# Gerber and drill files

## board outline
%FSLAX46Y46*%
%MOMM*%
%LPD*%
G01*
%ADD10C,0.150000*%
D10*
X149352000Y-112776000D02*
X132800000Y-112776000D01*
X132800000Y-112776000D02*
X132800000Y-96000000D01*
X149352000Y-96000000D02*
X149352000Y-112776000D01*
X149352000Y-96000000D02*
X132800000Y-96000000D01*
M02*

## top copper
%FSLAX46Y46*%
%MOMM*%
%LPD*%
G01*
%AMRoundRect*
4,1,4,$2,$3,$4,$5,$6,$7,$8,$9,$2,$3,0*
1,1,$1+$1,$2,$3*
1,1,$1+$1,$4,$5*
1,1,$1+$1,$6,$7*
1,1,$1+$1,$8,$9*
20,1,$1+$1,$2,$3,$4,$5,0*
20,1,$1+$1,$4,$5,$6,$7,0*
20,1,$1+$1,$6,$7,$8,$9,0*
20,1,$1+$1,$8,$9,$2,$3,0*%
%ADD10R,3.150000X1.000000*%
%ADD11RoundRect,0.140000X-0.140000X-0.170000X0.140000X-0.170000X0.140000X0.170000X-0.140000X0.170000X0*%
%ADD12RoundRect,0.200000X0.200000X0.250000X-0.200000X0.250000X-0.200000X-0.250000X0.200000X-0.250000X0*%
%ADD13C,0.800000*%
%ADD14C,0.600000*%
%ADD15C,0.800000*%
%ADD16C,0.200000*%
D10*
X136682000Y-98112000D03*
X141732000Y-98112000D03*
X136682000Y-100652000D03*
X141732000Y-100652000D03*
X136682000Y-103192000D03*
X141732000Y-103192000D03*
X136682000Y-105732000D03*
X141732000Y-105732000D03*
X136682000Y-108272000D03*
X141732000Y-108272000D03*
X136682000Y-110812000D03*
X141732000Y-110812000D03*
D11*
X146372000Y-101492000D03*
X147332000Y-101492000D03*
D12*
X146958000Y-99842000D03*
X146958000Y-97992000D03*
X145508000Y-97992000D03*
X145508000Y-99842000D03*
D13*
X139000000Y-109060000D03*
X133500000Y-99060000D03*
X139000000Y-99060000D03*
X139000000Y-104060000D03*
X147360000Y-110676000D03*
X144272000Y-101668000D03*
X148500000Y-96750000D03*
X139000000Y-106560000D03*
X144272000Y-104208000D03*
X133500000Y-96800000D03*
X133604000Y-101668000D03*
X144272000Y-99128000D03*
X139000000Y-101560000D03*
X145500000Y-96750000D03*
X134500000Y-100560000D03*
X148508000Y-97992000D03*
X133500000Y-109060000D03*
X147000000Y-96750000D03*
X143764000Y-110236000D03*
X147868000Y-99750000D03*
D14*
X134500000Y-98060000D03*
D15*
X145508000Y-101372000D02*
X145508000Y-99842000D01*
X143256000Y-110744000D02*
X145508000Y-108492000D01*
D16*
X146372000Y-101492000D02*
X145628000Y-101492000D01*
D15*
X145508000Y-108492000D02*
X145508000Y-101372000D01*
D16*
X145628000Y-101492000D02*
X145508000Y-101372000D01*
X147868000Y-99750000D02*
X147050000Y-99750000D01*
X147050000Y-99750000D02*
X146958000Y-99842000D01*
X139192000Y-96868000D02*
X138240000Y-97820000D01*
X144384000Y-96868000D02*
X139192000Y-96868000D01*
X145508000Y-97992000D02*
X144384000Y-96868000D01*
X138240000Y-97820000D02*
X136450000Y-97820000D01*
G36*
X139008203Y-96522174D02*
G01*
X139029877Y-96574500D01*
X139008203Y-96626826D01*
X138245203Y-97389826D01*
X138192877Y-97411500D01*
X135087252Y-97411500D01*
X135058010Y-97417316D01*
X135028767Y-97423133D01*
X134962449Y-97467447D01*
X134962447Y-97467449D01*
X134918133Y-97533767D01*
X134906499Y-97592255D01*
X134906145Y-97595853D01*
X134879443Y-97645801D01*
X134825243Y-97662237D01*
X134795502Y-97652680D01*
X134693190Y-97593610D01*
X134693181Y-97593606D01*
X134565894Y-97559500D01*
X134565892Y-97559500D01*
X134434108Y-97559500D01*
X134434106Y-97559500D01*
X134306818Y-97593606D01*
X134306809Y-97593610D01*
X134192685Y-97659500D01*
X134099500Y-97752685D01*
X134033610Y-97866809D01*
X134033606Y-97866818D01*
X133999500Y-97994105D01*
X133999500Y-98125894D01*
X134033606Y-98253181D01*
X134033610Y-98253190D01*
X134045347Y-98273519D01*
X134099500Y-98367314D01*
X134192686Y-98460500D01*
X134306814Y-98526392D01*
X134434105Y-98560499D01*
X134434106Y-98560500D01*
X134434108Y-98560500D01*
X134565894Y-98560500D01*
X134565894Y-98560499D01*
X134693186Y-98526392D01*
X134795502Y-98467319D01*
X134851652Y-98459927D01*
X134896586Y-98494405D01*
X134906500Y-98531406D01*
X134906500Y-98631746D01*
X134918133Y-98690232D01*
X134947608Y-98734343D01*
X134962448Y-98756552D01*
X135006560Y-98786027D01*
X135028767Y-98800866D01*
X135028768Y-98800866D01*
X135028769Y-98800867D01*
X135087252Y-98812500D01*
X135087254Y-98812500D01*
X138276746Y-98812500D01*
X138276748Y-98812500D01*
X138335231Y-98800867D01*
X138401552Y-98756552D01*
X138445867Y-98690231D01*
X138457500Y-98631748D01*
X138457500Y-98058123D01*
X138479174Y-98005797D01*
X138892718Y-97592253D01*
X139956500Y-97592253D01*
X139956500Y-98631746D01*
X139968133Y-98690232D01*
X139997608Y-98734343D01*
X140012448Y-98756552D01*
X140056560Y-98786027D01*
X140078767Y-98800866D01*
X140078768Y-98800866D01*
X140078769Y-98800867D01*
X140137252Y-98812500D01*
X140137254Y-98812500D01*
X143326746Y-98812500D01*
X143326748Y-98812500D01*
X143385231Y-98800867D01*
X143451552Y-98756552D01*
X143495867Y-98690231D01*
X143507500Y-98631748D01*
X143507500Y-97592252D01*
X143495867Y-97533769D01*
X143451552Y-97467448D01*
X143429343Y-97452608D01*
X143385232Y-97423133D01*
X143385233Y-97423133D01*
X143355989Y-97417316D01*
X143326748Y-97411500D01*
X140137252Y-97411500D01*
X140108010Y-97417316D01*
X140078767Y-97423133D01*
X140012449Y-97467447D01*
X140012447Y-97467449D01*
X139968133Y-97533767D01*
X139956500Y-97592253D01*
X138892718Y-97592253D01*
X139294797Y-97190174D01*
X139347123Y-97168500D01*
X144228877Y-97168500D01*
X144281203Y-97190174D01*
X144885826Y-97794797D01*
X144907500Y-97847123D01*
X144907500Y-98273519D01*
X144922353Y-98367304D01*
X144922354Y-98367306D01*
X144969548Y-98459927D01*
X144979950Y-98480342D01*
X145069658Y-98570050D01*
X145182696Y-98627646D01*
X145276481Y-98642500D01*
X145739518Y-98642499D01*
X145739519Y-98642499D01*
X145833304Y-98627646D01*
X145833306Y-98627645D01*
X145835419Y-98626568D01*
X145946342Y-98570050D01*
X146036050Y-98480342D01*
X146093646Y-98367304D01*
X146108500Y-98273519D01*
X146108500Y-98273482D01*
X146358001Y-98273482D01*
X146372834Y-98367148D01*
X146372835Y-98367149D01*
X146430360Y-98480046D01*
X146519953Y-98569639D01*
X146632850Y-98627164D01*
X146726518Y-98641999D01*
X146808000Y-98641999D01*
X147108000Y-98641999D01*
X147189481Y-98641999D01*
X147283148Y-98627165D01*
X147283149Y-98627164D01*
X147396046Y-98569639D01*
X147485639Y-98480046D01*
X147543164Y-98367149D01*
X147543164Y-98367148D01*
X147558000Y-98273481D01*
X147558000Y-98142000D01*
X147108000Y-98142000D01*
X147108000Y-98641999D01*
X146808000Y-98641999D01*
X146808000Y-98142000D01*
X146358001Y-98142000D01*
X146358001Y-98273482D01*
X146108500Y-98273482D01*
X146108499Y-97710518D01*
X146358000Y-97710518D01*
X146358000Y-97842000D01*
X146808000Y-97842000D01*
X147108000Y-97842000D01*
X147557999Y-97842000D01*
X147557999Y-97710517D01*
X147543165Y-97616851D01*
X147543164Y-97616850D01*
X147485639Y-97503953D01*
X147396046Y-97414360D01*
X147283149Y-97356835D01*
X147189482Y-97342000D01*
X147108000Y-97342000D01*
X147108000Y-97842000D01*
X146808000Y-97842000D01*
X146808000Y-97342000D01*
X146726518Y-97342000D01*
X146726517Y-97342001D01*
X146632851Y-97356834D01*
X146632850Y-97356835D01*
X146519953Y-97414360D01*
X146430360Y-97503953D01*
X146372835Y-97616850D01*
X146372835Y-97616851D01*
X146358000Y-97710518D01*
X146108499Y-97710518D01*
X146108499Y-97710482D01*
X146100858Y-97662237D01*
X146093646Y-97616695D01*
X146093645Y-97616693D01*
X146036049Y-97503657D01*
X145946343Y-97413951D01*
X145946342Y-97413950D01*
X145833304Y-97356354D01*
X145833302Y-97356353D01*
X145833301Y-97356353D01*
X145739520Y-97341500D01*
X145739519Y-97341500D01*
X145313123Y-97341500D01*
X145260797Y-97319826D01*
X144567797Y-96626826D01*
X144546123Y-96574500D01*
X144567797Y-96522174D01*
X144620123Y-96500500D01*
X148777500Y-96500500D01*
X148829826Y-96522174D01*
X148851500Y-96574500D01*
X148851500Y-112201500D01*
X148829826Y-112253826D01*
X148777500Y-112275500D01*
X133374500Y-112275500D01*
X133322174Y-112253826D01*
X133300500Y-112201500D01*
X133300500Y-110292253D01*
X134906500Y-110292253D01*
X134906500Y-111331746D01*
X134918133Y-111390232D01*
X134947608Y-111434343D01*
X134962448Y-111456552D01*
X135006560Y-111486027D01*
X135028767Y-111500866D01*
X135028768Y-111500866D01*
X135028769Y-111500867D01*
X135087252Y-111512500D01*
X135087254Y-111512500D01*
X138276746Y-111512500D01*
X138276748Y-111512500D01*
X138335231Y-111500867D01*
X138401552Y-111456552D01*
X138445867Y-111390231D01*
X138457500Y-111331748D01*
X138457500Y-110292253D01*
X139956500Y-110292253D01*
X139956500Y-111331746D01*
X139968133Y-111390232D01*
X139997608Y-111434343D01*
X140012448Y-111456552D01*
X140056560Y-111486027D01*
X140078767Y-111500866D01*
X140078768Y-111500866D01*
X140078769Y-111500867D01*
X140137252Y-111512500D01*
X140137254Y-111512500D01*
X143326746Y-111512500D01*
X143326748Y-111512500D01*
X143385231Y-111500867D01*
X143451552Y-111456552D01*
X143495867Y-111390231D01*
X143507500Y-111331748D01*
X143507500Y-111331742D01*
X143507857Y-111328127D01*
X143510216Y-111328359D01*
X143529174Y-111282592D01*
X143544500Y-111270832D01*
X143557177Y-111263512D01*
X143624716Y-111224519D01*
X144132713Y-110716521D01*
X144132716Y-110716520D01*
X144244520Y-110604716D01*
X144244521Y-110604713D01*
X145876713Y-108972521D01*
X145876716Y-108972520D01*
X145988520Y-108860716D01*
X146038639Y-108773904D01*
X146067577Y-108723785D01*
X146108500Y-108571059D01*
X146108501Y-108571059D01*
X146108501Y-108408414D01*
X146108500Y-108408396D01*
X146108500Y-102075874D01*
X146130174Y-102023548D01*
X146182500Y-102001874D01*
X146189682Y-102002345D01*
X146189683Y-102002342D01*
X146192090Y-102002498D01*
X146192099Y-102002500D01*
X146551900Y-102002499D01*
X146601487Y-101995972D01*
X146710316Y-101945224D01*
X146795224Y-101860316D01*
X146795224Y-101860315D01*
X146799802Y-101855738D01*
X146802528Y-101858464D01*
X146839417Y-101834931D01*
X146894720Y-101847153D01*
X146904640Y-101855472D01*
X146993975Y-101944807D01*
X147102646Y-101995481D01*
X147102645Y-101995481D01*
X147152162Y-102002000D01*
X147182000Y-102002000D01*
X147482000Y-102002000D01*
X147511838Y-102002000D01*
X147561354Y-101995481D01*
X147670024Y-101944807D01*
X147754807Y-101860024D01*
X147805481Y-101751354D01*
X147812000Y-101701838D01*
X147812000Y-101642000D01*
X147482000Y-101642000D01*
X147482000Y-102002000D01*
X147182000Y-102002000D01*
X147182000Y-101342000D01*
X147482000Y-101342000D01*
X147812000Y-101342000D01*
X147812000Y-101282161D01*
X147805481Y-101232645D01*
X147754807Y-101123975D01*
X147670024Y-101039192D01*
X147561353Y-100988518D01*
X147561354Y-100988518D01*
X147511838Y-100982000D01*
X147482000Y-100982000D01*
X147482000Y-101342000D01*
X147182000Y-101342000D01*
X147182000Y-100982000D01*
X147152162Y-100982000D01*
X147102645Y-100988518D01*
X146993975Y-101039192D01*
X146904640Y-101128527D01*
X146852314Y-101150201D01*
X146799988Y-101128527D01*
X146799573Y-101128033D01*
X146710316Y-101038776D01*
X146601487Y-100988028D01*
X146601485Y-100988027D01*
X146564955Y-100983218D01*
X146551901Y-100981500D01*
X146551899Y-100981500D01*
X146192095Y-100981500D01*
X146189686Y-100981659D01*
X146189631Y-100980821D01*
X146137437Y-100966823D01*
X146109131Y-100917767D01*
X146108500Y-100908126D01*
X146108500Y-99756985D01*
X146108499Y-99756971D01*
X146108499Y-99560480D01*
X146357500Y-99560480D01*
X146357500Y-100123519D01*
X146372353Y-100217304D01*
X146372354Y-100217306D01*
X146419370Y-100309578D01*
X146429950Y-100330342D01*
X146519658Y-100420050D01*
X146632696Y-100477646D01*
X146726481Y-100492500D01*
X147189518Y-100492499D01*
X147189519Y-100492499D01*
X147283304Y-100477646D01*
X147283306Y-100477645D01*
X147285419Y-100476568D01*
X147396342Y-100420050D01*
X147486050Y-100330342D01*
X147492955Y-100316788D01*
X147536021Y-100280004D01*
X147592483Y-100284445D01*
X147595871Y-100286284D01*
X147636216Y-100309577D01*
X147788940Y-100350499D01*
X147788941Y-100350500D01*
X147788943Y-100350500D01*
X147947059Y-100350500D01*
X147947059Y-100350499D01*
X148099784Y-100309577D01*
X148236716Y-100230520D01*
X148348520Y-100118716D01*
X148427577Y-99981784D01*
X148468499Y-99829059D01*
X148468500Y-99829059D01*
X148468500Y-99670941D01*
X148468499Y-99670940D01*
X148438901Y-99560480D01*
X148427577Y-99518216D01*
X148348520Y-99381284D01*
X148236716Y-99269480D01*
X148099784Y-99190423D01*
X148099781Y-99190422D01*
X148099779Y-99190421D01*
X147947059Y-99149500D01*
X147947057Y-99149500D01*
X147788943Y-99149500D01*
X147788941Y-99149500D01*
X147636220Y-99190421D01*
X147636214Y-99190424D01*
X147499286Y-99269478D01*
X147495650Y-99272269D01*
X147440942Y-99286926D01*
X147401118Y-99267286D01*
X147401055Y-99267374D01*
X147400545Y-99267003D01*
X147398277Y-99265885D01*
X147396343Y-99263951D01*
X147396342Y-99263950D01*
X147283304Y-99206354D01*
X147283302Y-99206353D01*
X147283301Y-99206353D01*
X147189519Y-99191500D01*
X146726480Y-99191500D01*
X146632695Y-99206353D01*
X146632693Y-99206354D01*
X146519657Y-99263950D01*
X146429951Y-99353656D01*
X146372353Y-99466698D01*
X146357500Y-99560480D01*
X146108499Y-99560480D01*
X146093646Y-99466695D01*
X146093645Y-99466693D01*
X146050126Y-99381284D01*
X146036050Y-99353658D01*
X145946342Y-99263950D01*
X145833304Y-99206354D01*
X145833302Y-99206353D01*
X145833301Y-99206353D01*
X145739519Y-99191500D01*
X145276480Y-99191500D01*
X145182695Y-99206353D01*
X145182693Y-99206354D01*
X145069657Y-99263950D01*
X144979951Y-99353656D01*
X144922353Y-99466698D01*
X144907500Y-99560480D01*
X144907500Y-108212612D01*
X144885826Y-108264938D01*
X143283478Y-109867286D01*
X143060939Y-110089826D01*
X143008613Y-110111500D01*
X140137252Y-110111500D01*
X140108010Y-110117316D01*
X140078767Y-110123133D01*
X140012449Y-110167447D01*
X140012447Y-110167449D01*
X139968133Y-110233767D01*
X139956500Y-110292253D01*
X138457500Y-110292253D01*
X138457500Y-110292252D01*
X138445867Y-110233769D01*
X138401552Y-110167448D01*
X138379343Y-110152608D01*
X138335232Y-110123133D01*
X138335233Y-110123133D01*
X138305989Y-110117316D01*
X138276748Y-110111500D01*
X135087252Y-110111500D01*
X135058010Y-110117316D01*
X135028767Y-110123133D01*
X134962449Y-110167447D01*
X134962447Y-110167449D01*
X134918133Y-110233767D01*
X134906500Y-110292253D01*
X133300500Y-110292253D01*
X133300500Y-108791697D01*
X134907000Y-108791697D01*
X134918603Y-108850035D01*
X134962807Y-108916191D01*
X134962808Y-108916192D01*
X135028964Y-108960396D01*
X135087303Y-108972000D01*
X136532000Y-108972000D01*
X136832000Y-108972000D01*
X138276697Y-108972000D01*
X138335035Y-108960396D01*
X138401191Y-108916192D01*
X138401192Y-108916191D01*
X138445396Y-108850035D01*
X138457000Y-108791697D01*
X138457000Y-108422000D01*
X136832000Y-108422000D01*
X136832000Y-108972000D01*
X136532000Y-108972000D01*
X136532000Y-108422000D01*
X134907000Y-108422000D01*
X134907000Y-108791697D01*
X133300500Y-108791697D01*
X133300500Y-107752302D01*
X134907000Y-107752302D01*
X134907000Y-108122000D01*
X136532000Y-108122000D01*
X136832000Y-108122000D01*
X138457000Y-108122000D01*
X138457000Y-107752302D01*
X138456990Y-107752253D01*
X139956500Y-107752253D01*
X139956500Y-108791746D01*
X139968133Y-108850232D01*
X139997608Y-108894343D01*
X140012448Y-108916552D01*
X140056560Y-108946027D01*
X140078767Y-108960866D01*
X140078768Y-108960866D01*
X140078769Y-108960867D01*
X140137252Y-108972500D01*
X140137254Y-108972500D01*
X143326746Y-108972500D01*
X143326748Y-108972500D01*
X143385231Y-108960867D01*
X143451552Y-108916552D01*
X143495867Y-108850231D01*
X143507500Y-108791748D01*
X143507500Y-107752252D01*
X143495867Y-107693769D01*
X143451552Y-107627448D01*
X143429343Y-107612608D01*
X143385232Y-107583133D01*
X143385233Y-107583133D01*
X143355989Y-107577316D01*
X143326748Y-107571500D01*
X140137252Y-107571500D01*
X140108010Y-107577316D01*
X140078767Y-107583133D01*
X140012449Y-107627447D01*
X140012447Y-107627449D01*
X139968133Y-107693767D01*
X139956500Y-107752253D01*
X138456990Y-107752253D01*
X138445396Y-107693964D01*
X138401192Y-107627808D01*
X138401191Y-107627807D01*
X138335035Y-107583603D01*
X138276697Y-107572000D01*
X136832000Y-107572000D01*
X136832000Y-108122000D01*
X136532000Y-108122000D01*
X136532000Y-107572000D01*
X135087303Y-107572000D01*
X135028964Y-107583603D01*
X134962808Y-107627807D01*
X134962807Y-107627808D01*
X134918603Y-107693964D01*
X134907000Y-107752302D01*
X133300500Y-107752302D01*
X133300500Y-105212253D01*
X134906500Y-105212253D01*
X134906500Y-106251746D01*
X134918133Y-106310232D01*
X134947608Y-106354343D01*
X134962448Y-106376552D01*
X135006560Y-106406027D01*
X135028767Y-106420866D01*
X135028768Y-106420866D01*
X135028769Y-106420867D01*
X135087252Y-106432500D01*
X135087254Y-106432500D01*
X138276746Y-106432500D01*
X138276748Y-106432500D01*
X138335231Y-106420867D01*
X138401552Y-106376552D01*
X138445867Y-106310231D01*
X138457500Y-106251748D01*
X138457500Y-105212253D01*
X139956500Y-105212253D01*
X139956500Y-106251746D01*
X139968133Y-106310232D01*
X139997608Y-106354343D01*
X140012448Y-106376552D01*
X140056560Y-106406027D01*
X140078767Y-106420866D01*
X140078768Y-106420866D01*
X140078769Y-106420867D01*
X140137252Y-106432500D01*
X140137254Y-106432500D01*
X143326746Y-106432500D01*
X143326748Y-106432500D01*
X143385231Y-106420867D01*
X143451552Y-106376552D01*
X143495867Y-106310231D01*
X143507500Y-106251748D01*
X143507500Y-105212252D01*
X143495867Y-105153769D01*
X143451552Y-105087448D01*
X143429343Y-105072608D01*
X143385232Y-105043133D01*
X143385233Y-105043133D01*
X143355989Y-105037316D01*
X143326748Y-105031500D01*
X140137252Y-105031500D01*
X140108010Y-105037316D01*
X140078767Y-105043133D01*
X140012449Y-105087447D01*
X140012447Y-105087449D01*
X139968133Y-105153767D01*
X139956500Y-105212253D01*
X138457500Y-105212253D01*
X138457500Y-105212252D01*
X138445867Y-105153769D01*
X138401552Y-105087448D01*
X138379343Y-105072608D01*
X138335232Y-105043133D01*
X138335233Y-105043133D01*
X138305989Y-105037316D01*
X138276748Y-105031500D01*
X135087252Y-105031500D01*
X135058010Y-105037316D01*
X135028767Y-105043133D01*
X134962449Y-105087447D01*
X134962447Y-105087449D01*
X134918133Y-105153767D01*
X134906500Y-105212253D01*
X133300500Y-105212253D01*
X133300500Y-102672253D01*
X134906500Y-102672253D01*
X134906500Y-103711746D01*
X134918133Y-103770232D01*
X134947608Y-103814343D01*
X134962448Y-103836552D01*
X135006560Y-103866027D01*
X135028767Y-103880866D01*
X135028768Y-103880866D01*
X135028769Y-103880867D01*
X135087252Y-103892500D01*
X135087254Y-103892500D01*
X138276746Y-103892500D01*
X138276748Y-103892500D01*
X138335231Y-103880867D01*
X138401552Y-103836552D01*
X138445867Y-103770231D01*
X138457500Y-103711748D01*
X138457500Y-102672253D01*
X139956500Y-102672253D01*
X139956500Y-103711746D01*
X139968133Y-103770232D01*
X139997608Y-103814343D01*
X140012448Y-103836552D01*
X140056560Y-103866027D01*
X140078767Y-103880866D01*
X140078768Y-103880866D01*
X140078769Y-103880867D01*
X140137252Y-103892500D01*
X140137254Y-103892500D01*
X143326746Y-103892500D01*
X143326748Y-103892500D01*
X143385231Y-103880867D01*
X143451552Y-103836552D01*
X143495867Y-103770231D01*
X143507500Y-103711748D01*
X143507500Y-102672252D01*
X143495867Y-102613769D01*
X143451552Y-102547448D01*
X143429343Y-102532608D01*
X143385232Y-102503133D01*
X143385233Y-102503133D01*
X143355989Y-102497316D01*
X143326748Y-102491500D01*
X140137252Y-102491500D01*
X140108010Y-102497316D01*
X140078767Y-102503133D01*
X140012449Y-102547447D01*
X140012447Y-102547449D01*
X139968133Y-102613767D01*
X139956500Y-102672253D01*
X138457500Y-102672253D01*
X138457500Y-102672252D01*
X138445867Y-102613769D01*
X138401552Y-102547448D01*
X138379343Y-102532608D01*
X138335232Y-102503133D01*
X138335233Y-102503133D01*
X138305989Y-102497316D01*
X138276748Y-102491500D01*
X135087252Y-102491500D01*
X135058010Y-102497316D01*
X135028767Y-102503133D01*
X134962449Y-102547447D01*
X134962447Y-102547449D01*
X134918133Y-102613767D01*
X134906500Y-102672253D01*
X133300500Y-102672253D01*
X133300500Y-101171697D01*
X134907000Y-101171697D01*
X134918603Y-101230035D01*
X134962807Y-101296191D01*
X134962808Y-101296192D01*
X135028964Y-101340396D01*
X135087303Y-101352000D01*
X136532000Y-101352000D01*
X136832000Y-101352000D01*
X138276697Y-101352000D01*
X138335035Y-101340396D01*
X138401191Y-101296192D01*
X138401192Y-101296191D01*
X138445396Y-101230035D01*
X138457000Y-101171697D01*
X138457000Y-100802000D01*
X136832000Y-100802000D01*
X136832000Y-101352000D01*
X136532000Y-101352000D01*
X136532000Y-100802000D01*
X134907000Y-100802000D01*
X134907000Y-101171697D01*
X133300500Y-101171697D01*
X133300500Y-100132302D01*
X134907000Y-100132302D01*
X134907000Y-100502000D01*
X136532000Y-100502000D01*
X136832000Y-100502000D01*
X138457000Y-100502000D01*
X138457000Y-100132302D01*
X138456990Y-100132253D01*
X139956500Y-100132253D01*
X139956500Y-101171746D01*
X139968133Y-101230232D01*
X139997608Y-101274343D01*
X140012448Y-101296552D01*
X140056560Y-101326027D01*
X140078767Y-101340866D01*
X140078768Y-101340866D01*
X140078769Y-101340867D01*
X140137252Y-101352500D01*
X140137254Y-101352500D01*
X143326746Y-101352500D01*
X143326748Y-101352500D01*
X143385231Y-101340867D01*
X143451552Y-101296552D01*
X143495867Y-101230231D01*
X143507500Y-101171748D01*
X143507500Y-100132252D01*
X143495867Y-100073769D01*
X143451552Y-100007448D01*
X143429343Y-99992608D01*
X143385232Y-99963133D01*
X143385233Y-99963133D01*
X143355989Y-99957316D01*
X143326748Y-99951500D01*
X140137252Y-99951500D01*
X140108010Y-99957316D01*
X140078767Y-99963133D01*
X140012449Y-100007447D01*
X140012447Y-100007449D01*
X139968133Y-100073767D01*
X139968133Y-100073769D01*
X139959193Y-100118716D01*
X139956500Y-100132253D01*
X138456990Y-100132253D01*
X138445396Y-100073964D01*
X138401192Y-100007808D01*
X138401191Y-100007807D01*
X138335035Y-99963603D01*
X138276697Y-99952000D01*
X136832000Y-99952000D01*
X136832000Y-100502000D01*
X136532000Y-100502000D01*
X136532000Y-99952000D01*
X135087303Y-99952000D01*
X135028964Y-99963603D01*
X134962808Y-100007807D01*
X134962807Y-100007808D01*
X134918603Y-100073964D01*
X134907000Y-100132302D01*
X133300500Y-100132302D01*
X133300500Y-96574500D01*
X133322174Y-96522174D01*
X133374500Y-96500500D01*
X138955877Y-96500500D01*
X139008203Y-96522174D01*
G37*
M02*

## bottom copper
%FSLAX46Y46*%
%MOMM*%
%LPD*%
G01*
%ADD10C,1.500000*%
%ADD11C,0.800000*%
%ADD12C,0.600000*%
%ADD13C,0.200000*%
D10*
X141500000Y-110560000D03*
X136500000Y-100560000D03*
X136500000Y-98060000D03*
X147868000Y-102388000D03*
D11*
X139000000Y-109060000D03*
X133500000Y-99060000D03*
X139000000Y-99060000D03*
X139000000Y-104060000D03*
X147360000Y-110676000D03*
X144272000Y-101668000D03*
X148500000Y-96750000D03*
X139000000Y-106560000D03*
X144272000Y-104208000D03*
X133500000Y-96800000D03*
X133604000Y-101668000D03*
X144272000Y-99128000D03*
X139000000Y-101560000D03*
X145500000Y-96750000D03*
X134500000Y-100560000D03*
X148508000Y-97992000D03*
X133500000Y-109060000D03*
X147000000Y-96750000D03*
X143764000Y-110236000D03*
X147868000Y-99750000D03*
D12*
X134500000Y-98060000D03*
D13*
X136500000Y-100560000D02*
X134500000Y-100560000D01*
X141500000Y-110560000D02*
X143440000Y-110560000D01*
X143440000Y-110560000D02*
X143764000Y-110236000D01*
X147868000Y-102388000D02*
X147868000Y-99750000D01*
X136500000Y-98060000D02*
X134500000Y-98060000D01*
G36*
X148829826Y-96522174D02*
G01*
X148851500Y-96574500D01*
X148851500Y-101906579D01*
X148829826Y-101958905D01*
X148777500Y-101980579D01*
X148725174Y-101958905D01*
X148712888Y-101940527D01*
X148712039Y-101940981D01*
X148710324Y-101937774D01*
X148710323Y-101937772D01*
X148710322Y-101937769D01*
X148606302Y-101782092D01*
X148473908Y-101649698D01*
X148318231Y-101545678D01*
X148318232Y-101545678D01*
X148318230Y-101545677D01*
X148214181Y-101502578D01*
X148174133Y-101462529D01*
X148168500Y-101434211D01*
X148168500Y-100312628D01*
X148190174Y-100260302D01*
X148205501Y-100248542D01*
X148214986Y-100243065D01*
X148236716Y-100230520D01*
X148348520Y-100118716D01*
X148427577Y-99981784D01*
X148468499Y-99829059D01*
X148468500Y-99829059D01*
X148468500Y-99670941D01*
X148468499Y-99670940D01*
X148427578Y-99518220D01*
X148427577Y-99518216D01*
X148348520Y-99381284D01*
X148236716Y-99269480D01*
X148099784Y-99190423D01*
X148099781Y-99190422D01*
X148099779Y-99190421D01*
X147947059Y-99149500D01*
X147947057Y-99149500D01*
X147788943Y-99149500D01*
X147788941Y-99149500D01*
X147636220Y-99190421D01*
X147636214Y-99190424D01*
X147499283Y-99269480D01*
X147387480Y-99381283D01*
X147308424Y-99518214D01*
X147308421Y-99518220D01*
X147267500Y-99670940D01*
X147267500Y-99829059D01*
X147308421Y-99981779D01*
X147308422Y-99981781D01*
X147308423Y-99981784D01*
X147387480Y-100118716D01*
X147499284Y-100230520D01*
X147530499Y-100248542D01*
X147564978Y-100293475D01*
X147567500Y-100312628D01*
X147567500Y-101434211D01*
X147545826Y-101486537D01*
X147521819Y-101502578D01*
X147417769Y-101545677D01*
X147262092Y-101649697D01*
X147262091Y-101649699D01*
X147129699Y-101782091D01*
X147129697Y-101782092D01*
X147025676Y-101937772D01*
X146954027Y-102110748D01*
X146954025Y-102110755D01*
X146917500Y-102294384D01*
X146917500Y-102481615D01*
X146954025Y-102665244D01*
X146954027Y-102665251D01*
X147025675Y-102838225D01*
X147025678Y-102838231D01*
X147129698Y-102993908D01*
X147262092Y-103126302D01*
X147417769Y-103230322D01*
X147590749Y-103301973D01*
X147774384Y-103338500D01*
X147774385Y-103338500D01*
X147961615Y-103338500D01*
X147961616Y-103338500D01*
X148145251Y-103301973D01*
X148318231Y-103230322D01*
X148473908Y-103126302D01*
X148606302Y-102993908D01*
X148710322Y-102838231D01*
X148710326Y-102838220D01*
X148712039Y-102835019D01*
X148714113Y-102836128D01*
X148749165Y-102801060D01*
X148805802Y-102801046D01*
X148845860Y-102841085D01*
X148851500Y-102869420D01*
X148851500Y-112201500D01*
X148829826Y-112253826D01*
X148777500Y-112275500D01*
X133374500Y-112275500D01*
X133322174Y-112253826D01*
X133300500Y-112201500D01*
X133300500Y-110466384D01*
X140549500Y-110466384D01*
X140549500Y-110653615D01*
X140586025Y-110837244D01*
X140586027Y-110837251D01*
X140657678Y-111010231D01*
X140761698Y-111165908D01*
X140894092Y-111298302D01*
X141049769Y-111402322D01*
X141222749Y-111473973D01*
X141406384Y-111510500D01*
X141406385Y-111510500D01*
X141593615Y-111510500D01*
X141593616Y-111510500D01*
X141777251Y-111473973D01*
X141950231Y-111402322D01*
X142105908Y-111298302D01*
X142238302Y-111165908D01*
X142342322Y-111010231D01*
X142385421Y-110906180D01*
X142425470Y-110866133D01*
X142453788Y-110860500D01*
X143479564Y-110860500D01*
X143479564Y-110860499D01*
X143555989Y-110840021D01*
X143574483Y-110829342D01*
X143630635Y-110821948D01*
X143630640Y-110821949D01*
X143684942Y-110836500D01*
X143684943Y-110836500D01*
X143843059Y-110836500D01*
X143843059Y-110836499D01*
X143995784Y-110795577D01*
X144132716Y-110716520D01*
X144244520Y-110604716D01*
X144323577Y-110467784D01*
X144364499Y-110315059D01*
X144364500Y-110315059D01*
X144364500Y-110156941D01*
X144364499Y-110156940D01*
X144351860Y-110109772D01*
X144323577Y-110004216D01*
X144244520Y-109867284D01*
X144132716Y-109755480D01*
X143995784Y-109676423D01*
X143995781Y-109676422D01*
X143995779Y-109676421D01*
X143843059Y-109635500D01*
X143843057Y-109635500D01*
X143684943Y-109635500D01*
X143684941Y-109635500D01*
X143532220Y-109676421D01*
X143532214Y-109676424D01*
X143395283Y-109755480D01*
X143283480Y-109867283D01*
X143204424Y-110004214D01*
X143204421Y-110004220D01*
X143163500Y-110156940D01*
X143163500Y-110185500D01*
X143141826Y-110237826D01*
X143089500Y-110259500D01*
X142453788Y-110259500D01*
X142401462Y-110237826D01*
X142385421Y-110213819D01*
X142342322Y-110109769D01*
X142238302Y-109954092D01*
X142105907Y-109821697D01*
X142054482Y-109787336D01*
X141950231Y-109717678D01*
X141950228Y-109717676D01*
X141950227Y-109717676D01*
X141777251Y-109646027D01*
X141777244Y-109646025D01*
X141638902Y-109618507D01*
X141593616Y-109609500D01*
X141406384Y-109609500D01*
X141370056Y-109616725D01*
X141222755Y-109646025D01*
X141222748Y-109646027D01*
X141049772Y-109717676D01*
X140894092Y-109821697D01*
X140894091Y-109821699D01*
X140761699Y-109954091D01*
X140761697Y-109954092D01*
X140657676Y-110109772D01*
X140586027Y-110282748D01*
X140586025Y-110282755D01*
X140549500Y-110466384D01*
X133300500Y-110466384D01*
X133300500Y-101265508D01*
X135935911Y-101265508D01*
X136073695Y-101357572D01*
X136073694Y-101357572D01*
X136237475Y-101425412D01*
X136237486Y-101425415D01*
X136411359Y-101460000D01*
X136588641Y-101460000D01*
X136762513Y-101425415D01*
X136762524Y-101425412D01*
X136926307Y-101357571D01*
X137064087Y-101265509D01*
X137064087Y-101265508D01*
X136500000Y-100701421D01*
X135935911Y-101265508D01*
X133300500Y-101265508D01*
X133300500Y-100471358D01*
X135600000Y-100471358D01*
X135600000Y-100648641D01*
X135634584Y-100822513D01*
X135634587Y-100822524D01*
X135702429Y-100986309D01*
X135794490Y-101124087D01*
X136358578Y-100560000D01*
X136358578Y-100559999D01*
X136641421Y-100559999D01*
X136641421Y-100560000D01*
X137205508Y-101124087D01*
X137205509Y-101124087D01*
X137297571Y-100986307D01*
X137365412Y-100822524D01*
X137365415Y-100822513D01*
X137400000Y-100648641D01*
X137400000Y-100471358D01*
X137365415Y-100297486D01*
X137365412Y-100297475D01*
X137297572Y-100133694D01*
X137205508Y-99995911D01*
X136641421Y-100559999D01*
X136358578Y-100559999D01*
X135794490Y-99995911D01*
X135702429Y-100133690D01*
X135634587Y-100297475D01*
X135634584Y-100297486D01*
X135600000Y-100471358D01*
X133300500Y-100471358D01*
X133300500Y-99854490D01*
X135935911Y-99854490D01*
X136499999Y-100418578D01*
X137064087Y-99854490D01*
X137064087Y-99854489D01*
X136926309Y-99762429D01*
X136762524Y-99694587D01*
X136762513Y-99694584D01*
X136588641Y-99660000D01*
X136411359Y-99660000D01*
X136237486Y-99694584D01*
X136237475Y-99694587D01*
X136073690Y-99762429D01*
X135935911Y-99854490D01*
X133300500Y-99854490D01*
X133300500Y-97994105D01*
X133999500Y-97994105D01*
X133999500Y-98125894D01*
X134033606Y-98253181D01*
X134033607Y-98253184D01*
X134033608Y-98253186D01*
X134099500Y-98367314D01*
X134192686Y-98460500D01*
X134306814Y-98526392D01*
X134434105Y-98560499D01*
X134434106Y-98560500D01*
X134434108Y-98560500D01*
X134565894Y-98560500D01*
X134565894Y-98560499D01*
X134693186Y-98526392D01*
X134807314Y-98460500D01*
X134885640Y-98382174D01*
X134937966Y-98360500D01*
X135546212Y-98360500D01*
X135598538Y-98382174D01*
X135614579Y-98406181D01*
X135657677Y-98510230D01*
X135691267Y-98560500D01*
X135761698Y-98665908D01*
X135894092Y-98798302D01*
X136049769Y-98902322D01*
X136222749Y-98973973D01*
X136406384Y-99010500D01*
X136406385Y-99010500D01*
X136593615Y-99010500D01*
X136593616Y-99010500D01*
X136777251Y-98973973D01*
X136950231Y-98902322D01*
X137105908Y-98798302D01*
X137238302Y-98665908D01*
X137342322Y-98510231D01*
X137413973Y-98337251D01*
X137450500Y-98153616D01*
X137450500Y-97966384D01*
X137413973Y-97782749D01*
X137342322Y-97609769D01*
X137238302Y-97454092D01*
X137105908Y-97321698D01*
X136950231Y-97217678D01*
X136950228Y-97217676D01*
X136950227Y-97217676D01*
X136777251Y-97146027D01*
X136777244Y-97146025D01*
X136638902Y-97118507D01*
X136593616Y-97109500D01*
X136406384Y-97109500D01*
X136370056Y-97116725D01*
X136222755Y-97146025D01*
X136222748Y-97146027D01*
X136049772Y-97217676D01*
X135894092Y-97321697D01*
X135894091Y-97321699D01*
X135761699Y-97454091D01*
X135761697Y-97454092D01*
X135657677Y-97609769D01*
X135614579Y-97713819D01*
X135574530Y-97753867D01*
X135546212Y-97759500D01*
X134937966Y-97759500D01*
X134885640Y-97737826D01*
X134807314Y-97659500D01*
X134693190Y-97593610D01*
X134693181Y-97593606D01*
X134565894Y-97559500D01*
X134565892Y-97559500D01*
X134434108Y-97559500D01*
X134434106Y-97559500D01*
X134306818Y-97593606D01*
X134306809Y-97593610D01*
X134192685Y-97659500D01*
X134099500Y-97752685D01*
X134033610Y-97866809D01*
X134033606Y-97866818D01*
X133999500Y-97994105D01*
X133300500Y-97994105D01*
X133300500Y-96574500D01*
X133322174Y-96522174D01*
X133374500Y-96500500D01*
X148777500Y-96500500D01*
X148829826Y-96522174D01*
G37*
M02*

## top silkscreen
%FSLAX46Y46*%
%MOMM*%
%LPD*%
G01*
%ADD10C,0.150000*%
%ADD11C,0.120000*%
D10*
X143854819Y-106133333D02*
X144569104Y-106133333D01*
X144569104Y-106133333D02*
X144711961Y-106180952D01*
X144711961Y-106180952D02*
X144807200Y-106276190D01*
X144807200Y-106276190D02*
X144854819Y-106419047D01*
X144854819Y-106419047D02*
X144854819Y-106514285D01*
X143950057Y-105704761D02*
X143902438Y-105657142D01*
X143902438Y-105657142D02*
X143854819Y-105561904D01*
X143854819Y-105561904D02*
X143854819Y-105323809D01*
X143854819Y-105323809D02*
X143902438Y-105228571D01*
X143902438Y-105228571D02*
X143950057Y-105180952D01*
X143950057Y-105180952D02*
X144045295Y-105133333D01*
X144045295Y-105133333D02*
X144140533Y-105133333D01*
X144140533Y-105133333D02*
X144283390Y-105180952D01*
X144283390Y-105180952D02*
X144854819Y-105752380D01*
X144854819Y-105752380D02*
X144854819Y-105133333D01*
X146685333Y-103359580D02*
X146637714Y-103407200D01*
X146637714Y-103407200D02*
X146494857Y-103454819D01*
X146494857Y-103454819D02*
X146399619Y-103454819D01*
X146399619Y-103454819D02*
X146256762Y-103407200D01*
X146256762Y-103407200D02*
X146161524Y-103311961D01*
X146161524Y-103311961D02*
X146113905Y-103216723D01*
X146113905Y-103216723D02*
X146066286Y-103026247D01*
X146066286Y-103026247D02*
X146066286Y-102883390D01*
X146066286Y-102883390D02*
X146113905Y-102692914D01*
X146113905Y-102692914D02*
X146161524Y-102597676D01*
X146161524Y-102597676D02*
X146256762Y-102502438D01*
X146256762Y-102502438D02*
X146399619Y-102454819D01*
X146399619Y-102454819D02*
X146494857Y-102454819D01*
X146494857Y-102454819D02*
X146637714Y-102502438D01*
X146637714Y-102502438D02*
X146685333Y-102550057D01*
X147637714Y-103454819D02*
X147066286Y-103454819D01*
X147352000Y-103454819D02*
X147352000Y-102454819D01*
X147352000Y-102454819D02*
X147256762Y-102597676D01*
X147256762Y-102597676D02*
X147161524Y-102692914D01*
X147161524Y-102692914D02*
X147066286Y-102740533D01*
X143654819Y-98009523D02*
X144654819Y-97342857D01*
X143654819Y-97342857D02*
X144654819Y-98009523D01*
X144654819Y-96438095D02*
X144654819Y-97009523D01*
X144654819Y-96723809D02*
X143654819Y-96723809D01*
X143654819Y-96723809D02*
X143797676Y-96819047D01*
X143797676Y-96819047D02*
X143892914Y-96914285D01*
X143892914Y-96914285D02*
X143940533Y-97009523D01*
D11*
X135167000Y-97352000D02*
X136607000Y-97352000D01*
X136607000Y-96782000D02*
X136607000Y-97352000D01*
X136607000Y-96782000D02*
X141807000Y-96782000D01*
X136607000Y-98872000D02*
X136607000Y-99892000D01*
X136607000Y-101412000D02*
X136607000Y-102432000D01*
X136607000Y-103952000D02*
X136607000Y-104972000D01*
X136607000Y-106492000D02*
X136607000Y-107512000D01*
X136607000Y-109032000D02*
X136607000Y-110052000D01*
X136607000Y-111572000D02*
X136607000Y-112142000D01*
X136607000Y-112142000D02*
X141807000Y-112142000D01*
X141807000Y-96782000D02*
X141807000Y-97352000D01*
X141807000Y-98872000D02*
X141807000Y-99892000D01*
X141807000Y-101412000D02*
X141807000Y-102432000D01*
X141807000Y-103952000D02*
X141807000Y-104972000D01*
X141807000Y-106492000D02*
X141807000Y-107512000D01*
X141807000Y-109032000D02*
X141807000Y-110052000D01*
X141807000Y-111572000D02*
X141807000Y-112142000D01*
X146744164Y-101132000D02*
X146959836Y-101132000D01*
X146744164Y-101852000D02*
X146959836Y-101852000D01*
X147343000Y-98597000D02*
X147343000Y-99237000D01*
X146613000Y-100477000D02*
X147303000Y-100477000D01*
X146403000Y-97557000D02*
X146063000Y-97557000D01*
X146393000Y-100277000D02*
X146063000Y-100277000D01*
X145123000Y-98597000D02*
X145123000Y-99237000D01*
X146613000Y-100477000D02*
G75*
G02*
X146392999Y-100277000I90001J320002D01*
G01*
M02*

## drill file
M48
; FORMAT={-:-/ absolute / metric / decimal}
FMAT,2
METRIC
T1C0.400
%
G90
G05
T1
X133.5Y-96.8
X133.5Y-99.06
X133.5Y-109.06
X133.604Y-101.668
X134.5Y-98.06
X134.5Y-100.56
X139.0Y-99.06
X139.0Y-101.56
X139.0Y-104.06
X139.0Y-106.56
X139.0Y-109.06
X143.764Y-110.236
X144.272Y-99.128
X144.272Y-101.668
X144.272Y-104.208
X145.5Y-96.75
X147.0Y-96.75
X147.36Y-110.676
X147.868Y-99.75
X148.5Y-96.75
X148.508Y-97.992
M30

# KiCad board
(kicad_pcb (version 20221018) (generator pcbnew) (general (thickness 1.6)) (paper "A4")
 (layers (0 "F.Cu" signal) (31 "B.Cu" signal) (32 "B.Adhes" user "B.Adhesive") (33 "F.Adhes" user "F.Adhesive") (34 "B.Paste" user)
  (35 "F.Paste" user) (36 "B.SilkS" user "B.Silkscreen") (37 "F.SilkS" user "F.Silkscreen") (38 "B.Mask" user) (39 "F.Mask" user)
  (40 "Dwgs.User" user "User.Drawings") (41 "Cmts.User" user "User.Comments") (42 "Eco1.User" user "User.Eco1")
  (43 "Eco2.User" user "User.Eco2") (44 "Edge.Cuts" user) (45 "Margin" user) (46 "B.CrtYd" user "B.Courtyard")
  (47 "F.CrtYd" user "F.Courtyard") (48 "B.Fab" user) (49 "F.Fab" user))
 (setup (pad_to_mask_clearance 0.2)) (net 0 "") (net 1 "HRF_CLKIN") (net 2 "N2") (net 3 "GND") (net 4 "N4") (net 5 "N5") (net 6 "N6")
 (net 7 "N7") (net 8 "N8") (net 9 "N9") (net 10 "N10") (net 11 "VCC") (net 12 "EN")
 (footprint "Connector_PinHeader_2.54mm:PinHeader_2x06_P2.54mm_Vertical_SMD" (layer "F.Cu") (at 139.207 104.462)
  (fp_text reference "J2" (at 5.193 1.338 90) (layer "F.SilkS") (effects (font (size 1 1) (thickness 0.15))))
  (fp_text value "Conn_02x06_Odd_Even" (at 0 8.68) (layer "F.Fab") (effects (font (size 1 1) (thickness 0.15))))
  (fp_line (start -4.04 -7.11) (end -2.6 -7.11) (stroke (width 0.12) (type solid)) (layer "F.SilkS"))
  (fp_line (start -2.6 -7.68) (end -2.6 -7.11) (stroke (width 0.12) (type solid)) (layer "F.SilkS"))
  (fp_line (start -2.6 -7.68) (end 2.6 -7.68) (stroke (width 0.12) (type solid)) (layer "F.SilkS"))
  (fp_line (start -2.6 -5.59) (end -2.6 -4.57) (stroke (width 0.12) (type solid)) (layer "F.SilkS"))
  (fp_line (start -2.6 -3.05) (end -2.6 -2.03) (stroke (width 0.12) (type solid)) (layer "F.SilkS"))
  (fp_line (start -2.6 -0.51) (end -2.6 0.51) (stroke (width 0.12) (type solid)) (layer "F.SilkS"))
  (fp_line (start -2.6 2.03) (end -2.6 3.05) (stroke (width 0.12) (type solid)) (layer "F.SilkS"))
  (fp_line (start -2.6 4.57) (end -2.6 5.59) (stroke (width 0.12) (type solid)) (layer "F.SilkS"))
  (fp_line (start -2.6 7.11) (end -2.6 7.68) (stroke (width 0.12) (type solid)) (layer "F.SilkS"))
  (fp_line (start -2.6 7.68) (end 2.6 7.68) (stroke (width 0.12) (type solid)) (layer "F.SilkS"))
  (fp_line (start 2.6 -7.68) (end 2.6 -7.11) (stroke (width 0.12) (type solid)) (layer "F.SilkS"))
  (fp_line (start 2.6 -5.59) (end 2.6 -4.57) (stroke (width 0.12) (type solid)) (layer "F.SilkS"))
  (fp_line (start 2.6 -3.05) (end 2.6 -2.03) (stroke (width 0.12) (type solid)) (layer "F.SilkS"))
  (fp_line (start 2.6 -0.51) (end 2.6 0.51) (stroke (width 0.12) (type solid)) (layer "F.SilkS"))
  (fp_line (start 2.6 2.03) (end 2.6 3.05) (stroke (width 0.12) (type solid)) (layer "F.SilkS"))
  (fp_line (start 2.6 4.57) (end 2.6 5.59) (stroke (width 0.12) (type solid)) (layer "F.SilkS"))
  (fp_line (start 2.6 7.11) (end 2.6 7.68) (stroke (width 0.12) (type solid)) (layer "F.SilkS"))
  (pad "1" smd rect (at -2.525 -6.35) (size 3.15 1) (layers "F.Cu" "F.Paste" "F.Mask") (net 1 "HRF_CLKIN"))
  (pad "2" smd rect (at 2.525 -6.35) (size 3.15 1) (layers "F.Cu" "F.Paste" "F.Mask") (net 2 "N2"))
  (pad "3" smd rect (at -2.525 -3.81) (size 3.15 1) (layers "F.Cu" "F.Paste" "F.Mask") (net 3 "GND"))
  (pad "4" smd rect (at 2.525 -3.81) (size 3.15 1) (layers "F.Cu" "F.Paste" "F.Mask") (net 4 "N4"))
  (pad "5" smd rect (at -2.525 -1.27) (size 3.15 1) (layers "F.Cu" "F.Paste" "F.Mask") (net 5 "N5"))
  (pad "6" smd rect (at 2.525 -1.27) (size 3.15 1) (layers "F.Cu" "F.Paste" "F.Mask") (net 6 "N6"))
  (pad "7" smd rect (at -2.525 1.27) (size 3.15 1) (layers "F.Cu" "F.Paste" "F.Mask") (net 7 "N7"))
  (pad "8" smd rect (at 2.525 1.27) (size 3.15 1) (layers "F.Cu" "F.Paste" "F.Mask") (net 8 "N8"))
  (pad "9" smd rect (at -2.525 3.81) (size 3.15 1) (layers "F.Cu" "F.Paste" "F.Mask") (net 3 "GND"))
  (pad "10" smd rect (at 2.525 3.81) (size 3.15 1) (layers "F.Cu" "F.Paste" "F.Mask") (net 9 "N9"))
  (pad "11" smd rect (at -2.525 6.35) (size 3.15 1) (layers "F.Cu" "F.Paste" "F.Mask") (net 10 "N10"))
  (pad "12" smd rect (at 2.525 6.35) (size 3.15 1) (layers "F.Cu" "F.Paste" "F.Mask") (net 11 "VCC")))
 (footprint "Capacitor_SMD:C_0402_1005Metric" (layer "F.Cu") (at 146.852 101.492)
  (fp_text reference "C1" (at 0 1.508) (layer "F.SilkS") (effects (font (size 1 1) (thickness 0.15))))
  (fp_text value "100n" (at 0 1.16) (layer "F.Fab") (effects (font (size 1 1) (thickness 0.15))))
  (fp_line (start -0.107836 -0.36) (end 0.107836 -0.36) (stroke (width 0.12) (type solid)) (layer "F.SilkS"))
  (fp_line (start -0.107836 0.36) (end 0.107836 0.36) (stroke (width 0.12) (type solid)) (layer "F.SilkS"))
  (pad "1" smd roundrect (at -0.48 0) (size 0.56 0.62) (layers "F.Cu" "F.Paste" "F.Mask") (roundrect_rratio 0.25) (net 11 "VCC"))
  (pad "2" smd roundrect (at 0.48 0) (size 0.56 0.62) (layers "F.Cu" "F.Paste" "F.Mask") (roundrect_rratio 0.25) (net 3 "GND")))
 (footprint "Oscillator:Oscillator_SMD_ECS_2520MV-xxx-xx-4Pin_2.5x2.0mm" (layer "F.Cu") (at 146.233 98.917 180)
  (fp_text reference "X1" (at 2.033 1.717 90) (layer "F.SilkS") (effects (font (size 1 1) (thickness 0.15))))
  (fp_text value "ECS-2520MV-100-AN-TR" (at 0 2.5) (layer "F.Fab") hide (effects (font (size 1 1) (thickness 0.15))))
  (fp_line (start -1.11 0.32) (end -1.11 -0.32) (stroke (width 0.12) (type solid)) (layer "F.SilkS"))
  (fp_line (start -0.38 -1.56) (end -1.07 -1.56) (stroke (width 0.12) (type solid)) (layer "F.SilkS"))
  (fp_line (start -0.17 1.36) (end 0.17 1.36) (stroke (width 0.12) (type solid)) (layer "F.SilkS"))
  (fp_line (start -0.16 -1.36) (end 0.17 -1.36) (stroke (width 0.12) (type solid)) (layer "F.SilkS"))
  (fp_line (start 1.11 0.32) (end 1.11 -0.32) (stroke (width 0.12) (type solid)) (layer "F.SilkS"))
  (fp_arc (start -0.38 -1.56) (mid -0.246393 -1.485967) (end -0.16 -1.36) (stroke (width 0.12) (type solid)) (layer "F.SilkS"))
  (pad "1" smd roundrect (at -0.725 -0.925 180) (size 0.8 0.9) (layers "F.Cu" "F.Paste" "F.Mask") (roundrect_rratio 0.25) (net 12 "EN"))
  (pad "2" smd roundrect (at -0.725 0.925 180) (size 0.8 0.9) (layers "F.Cu" "F.Paste" "F.Mask") (roundrect_rratio 0.25) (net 3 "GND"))
  (pad "3" smd roundrect (at 0.725 0.925 180) (size 0.8 0.9) (layers "F.Cu" "F.Paste" "F.Mask") (roundrect_rratio 0.25) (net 1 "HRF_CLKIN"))
  (pad "4" smd roundrect (at 0.725 -0.925 180) (size 0.8 0.9) (layers "F.Cu" "F.Paste" "F.Mask") (roundrect_rratio 0.25) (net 11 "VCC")))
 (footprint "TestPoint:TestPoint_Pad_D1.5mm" (layer "B.Cu") (at 141.5 110.56 180)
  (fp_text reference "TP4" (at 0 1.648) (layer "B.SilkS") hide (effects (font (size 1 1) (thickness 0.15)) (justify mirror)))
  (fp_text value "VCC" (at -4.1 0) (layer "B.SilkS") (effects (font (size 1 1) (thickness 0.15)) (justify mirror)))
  (pad "1" smd circle (at 0 0 180) (size 1.5 1.5) (layers "B.Cu" "B.Mask") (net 11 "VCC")))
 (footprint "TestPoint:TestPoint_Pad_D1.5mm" (layer "B.Cu") (at 136.5 100.56 180)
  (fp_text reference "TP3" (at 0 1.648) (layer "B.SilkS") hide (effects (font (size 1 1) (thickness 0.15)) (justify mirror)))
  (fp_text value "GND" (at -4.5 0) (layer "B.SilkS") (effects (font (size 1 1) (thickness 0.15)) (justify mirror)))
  (pad "1" smd circle (at 0 0 180) (size 1.5 1.5) (layers "B.Cu" "B.Mask") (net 3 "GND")))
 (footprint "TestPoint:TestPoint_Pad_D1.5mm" (layer "B.Cu") (at 136.5 98.06 180)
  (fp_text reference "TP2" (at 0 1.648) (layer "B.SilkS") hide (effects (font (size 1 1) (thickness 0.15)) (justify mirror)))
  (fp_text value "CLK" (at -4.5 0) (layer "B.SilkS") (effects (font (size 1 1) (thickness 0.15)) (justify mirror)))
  (pad "1" smd circle (at 0 0 180) (size 1.5 1.5) (layers "B.Cu" "B.Mask") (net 1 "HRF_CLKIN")))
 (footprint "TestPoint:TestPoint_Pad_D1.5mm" (layer "B.Cu") (at 147.868 102.388 180)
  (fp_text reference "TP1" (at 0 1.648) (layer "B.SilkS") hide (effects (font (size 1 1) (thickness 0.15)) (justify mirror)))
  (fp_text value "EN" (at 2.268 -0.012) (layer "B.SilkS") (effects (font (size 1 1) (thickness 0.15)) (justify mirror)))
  (pad "1" smd circle (at 0 0 180) (size 1.5 1.5) (layers "B.Cu" "B.Mask") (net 12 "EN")))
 (gr_line (start 149.352 112.776) (end 132.8 112.776) (stroke (width 0.15) (type solid)) (layer "Edge.Cuts"))
 (gr_line (start 132.8 112.776) (end 132.8 96) (stroke (width 0.15) (type solid)) (layer "Edge.Cuts"))
 (gr_line (start 149.352 96) (end 149.352 112.776) (stroke (width 0.15) (type solid)) (layer "Edge.Cuts"))
 (gr_line (start 149.352 96) (end 132.8 96) (stroke (width 0.15) (type solid)) (layer "Edge.Cuts"))
 (via (at 139 109.06) (size 0.8) (drill 0.4) (layers "F.Cu" "B.Cu") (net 3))
 (via (at 133.5 99.06) (size 0.8) (drill 0.4) (layers "F.Cu" "B.Cu") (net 3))
 (via (at 139 99.06) (size 0.8) (drill 0.4) (layers "F.Cu" "B.Cu") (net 3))
 (via (at 139 104.06) (size 0.8) (drill 0.4) (layers "F.Cu" "B.Cu") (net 3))
 (via (at 147.36 110.676) (size 0.8) (drill 0.4) (layers "F.Cu" "B.Cu") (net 3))
 (via (at 144.272 101.668) (size 0.8) (drill 0.4) (layers "F.Cu" "B.Cu") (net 3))
 (via (at 148.5 96.75) (size 0.8) (drill 0.4) (layers "F.Cu" "B.Cu") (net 3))
 (via (at 139 106.56) (size 0.8) (drill 0.4) (layers "F.Cu" "B.Cu") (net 3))
 (via (at 144.272 104.208) (size 0.8) (drill 0.4) (layers "F.Cu" "B.Cu") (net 3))
 (via (at 133.5 96.8) (size 0.8) (drill 0.4) (layers "F.Cu" "B.Cu") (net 3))
 (via (at 133.604 101.668) (size 0.8) (drill 0.4) (layers "F.Cu" "B.Cu") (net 3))
 (via (at 144.272 99.128) (size 0.8) (drill 0.4) (layers "F.Cu" "B.Cu") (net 3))
 (via (at 139 101.56) (size 0.8) (drill 0.4) (layers "F.Cu" "B.Cu") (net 3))
 (via (at 145.5 96.75) (size 0.8) (drill 0.4) (layers "F.Cu" "B.Cu") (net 3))
 (via (at 134.5 100.56) (size 0.8) (drill 0.4) (layers "F.Cu" "B.Cu") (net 3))
 (via (at 148.508 97.992) (size 0.8) (drill 0.4) (layers "F.Cu" "B.Cu") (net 3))
 (via (at 133.5 109.06) (size 0.8) (drill 0.4) (layers "F.Cu" "B.Cu") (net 3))
 (via (at 147 96.75) (size 0.8) (drill 0.4) (layers "F.Cu" "B.Cu") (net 3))
 (segment (start 136.5 100.56) (end 134.5 100.56) (width 0.2) (layer "B.Cu") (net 3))
 (segment (start 145.508 101.372) (end 145.508 99.842) (width 0.8) (layer "F.Cu") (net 11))
 (segment (start 143.256 110.744) (end 145.508 108.492) (width 0.8) (layer "F.Cu") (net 11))
 (segment (start 146.372 101.492) (end 145.628 101.492) (width 0.2) (layer "F.Cu") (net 11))
 (segment (start 145.508 108.492) (end 145.508 101.372) (width 0.8) (layer "F.Cu") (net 11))
 (segment (start 145.628 101.492) (end 145.508 101.372) (width 0.2) (layer "F.Cu") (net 11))
 (via (at 143.764 110.236) (size 0.8) (drill 0.4) (layers "F.Cu" "B.Cu") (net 11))
 (segment (start 141.5 110.56) (end 143.44 110.56) (width 0.2) (layer "B.Cu") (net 11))
 (segment (start 143.44 110.56) (end 143.764 110.236) (width 0.2) (layer "B.Cu") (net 11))
 (segment (start 147.868 99.75) (end 147.05 99.75) (width 0.2) (layer "F.Cu") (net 12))
 (segment (start 147.05 99.75) (end 146.958 99.842) (width 0.2) (layer "F.Cu") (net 12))
 (via (at 147.868 99.75) (size 0.8) (drill 0.4) (layers "F.Cu" "B.Cu") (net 12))
 (segment (start 147.868 102.388) (end 147.868 99.75) (width 0.2) (layer "B.Cu") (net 12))
 (segment (start 139.192 96.868) (end 138.24 97.82) (width 0.2) (layer "F.Cu") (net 1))
 (segment (start 144.384 96.868) (end 139.192 96.868) (width 0.2) (layer "F.Cu") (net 1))
 (segment (start 145.508 97.992) (end 144.384 96.868) (width 0.2) (layer "F.Cu") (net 1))
 (segment (start 138.24 97.82) (end 136.45 97.82) (width 0.2) (layer "F.Cu") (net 1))
 (via (at 134.5 98.06) (size 0.6) (drill 0.4) (layers "F.Cu" "B.Cu") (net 1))
 (segment (start 136.5 98.06) (end 134.5 98.06) (width 0.2) (layer "B.Cu") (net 1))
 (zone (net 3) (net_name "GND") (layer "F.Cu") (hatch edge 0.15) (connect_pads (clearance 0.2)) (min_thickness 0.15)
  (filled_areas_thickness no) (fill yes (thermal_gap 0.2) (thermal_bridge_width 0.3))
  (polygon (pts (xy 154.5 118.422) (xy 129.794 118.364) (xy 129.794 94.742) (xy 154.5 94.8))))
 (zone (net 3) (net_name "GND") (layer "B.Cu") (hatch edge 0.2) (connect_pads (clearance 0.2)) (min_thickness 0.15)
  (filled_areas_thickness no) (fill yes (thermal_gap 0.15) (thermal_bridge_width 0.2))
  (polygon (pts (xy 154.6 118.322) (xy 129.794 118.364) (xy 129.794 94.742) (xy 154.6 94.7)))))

